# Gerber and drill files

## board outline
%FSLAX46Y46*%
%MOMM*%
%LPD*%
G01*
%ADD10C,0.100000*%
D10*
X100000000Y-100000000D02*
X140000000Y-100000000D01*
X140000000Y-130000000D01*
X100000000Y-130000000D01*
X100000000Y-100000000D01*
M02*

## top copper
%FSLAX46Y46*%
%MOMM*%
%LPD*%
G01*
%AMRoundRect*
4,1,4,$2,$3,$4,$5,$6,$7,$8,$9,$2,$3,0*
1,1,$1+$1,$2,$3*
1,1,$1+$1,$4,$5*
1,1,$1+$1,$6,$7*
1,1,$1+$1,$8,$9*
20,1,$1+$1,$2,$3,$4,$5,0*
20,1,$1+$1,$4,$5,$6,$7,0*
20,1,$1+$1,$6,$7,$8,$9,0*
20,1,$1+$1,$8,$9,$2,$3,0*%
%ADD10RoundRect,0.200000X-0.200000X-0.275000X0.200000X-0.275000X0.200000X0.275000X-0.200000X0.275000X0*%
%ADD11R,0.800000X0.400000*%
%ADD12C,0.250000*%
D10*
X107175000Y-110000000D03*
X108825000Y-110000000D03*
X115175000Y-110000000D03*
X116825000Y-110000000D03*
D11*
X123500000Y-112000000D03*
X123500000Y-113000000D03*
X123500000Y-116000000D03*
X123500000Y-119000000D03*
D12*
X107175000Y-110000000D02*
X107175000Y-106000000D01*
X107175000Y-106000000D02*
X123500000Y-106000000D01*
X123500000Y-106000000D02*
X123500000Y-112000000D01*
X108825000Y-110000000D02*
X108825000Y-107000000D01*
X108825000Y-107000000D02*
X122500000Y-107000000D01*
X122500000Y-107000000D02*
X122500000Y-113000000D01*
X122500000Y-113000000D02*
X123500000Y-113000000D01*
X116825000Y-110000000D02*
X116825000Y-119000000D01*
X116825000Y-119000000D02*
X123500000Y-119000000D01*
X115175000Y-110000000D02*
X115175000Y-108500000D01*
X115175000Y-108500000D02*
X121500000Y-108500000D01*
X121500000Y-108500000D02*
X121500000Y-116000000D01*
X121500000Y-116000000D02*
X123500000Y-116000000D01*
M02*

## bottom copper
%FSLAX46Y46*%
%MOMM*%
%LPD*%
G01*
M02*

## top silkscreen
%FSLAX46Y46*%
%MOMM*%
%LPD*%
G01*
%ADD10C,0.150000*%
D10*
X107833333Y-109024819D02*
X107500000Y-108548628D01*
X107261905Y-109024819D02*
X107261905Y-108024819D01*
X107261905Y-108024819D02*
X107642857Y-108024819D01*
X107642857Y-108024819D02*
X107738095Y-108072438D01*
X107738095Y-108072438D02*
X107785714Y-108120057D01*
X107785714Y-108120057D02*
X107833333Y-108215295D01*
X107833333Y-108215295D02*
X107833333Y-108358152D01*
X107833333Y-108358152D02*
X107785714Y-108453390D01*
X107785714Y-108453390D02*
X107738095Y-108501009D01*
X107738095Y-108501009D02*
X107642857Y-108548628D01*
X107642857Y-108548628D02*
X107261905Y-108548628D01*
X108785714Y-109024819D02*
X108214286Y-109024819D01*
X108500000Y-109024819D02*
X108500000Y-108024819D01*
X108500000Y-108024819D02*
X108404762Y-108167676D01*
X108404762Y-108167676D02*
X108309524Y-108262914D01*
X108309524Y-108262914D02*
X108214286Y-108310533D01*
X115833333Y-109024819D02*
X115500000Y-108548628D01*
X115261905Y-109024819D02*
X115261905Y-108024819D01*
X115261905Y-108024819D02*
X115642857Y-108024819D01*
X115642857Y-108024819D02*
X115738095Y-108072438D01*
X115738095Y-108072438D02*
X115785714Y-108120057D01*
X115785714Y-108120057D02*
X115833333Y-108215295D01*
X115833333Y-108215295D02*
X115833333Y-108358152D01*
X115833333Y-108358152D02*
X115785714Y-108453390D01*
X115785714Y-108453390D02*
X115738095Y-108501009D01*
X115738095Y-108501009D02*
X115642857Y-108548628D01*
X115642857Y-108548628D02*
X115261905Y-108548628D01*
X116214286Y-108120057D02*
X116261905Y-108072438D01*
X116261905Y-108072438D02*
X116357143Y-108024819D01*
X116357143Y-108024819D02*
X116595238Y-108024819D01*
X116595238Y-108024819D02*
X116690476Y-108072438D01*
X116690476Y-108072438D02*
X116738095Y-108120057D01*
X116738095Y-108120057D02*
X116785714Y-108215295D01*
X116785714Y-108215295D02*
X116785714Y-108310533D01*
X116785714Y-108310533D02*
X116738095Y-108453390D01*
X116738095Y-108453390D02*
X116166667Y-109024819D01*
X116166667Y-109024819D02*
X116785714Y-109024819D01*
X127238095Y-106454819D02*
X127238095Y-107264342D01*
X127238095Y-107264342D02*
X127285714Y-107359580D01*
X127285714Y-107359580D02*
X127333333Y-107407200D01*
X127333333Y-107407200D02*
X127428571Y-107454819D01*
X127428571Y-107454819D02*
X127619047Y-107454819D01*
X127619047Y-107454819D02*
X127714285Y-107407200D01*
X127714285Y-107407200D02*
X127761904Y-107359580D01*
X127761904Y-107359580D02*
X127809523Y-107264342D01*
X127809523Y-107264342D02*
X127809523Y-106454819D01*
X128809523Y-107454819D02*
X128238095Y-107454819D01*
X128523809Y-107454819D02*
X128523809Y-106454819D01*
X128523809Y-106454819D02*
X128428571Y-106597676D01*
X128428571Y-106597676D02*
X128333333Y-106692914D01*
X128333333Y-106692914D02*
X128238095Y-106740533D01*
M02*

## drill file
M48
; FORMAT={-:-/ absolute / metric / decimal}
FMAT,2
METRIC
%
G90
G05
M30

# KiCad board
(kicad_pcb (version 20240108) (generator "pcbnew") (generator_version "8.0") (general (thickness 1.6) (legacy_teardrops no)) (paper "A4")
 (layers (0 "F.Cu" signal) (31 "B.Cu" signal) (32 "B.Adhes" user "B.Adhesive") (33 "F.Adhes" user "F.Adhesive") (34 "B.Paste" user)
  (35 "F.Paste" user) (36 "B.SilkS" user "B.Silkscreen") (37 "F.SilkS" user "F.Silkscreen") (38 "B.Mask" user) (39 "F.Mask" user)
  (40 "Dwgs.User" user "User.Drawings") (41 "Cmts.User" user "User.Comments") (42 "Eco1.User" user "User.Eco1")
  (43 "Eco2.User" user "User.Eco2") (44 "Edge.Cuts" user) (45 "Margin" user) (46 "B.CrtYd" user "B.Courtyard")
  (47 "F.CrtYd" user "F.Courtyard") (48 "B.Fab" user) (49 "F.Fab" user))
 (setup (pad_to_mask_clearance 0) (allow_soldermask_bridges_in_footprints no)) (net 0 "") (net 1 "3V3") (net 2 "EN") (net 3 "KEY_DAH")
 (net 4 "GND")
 (gr_rect (start 100 100) (end 140 130) (stroke (width 0.1) (type default)) (layer "Edge.Cuts"))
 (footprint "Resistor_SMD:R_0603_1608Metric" (layer "F.Cu") (at 108 110)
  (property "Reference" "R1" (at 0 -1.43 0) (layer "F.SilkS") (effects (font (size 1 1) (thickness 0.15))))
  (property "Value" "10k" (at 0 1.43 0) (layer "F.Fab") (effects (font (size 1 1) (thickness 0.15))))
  (pad "1" smd roundrect (at -0.825 0) (size 0.8 0.95) (layers "F.Cu" "F.Paste" "F.Mask") (roundrect_rratio 0.25) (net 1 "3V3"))
  (pad "2" smd roundrect (at 0.825 0) (size 0.8 0.95) (layers "F.Cu" "F.Paste" "F.Mask") (roundrect_rratio 0.25) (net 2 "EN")))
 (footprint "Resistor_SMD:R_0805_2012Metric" (layer "F.Cu") (at 116 110)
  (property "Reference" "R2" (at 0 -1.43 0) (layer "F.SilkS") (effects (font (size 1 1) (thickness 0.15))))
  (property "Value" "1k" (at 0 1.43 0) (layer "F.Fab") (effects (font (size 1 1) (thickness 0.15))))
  (pad "1" smd roundrect (at -0.825 0) (size 0.8 0.95) (layers "F.Cu" "F.Paste" "F.Mask") (roundrect_rratio 0.25) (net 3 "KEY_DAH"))
  (pad "2" smd roundrect (at 0.825 0) (size 0.8 0.95) (layers "F.Cu" "F.Paste" "F.Mask") (roundrect_rratio 0.25) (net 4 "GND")))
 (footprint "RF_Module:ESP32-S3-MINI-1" (layer "F.Cu") (at 128 115)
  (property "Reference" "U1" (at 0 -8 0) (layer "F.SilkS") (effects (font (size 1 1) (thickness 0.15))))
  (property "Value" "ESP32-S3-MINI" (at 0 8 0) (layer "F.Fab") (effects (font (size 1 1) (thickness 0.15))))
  (pad "1" smd rect (at -4.5 -3.0) (size 0.8 0.4) (layers "F.Cu" "F.Paste" "F.Mask") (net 1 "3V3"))
  (pad "2" smd rect (at -4.5 -2.0) (size 0.8 0.4) (layers "F.Cu" "F.Paste" "F.Mask") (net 2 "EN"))
  (pad "5" smd rect (at -4.5 1.0) (size 0.8 0.4) (layers "F.Cu" "F.Paste" "F.Mask") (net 3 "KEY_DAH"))
  (pad "8" smd rect (at -4.5 4.0) (size 0.8 0.4) (layers "F.Cu" "F.Paste" "F.Mask") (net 4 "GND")))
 (segment (start 107.175 110) (end 107.175 106) (width 0.25) (layer "F.Cu") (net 1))
 (segment (start 107.175 106) (end 123.5 106) (width 0.25) (layer "F.Cu") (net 1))
 (segment (start 123.5 106) (end 123.5 112) (width 0.25) (layer "F.Cu") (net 1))
 (segment (start 108.825 110) (end 108.825 107) (width 0.25) (layer "F.Cu") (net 2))
 (segment (start 108.825 107) (end 122.5 107) (width 0.25) (layer "F.Cu") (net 2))
 (segment (start 122.5 107) (end 122.5 113) (width 0.25) (layer "F.Cu") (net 2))
 (segment (start 122.5 113) (end 123.5 113) (width 0.25) (layer "F.Cu") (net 2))
 (segment (start 116.825 110) (end 116.825 119) (width 0.25) (layer "F.Cu") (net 4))
 (segment (start 116.825 119) (end 123.5 119) (width 0.25) (layer "F.Cu") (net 4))
 (segment (start 115.175 110) (end 115.175 108.5) (width 0.25) (layer "F.Cu") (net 3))
 (segment (start 115.175 108.5) (end 121.5 108.5) (width 0.25) (layer "F.Cu") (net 3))
 (segment (start 121.5 108.5) (end 121.5 116) (width 0.25) (layer "F.Cu") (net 3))
 (segment (start 121.5 116) (end 123.5 116) (width 0.25) (layer "F.Cu") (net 3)))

